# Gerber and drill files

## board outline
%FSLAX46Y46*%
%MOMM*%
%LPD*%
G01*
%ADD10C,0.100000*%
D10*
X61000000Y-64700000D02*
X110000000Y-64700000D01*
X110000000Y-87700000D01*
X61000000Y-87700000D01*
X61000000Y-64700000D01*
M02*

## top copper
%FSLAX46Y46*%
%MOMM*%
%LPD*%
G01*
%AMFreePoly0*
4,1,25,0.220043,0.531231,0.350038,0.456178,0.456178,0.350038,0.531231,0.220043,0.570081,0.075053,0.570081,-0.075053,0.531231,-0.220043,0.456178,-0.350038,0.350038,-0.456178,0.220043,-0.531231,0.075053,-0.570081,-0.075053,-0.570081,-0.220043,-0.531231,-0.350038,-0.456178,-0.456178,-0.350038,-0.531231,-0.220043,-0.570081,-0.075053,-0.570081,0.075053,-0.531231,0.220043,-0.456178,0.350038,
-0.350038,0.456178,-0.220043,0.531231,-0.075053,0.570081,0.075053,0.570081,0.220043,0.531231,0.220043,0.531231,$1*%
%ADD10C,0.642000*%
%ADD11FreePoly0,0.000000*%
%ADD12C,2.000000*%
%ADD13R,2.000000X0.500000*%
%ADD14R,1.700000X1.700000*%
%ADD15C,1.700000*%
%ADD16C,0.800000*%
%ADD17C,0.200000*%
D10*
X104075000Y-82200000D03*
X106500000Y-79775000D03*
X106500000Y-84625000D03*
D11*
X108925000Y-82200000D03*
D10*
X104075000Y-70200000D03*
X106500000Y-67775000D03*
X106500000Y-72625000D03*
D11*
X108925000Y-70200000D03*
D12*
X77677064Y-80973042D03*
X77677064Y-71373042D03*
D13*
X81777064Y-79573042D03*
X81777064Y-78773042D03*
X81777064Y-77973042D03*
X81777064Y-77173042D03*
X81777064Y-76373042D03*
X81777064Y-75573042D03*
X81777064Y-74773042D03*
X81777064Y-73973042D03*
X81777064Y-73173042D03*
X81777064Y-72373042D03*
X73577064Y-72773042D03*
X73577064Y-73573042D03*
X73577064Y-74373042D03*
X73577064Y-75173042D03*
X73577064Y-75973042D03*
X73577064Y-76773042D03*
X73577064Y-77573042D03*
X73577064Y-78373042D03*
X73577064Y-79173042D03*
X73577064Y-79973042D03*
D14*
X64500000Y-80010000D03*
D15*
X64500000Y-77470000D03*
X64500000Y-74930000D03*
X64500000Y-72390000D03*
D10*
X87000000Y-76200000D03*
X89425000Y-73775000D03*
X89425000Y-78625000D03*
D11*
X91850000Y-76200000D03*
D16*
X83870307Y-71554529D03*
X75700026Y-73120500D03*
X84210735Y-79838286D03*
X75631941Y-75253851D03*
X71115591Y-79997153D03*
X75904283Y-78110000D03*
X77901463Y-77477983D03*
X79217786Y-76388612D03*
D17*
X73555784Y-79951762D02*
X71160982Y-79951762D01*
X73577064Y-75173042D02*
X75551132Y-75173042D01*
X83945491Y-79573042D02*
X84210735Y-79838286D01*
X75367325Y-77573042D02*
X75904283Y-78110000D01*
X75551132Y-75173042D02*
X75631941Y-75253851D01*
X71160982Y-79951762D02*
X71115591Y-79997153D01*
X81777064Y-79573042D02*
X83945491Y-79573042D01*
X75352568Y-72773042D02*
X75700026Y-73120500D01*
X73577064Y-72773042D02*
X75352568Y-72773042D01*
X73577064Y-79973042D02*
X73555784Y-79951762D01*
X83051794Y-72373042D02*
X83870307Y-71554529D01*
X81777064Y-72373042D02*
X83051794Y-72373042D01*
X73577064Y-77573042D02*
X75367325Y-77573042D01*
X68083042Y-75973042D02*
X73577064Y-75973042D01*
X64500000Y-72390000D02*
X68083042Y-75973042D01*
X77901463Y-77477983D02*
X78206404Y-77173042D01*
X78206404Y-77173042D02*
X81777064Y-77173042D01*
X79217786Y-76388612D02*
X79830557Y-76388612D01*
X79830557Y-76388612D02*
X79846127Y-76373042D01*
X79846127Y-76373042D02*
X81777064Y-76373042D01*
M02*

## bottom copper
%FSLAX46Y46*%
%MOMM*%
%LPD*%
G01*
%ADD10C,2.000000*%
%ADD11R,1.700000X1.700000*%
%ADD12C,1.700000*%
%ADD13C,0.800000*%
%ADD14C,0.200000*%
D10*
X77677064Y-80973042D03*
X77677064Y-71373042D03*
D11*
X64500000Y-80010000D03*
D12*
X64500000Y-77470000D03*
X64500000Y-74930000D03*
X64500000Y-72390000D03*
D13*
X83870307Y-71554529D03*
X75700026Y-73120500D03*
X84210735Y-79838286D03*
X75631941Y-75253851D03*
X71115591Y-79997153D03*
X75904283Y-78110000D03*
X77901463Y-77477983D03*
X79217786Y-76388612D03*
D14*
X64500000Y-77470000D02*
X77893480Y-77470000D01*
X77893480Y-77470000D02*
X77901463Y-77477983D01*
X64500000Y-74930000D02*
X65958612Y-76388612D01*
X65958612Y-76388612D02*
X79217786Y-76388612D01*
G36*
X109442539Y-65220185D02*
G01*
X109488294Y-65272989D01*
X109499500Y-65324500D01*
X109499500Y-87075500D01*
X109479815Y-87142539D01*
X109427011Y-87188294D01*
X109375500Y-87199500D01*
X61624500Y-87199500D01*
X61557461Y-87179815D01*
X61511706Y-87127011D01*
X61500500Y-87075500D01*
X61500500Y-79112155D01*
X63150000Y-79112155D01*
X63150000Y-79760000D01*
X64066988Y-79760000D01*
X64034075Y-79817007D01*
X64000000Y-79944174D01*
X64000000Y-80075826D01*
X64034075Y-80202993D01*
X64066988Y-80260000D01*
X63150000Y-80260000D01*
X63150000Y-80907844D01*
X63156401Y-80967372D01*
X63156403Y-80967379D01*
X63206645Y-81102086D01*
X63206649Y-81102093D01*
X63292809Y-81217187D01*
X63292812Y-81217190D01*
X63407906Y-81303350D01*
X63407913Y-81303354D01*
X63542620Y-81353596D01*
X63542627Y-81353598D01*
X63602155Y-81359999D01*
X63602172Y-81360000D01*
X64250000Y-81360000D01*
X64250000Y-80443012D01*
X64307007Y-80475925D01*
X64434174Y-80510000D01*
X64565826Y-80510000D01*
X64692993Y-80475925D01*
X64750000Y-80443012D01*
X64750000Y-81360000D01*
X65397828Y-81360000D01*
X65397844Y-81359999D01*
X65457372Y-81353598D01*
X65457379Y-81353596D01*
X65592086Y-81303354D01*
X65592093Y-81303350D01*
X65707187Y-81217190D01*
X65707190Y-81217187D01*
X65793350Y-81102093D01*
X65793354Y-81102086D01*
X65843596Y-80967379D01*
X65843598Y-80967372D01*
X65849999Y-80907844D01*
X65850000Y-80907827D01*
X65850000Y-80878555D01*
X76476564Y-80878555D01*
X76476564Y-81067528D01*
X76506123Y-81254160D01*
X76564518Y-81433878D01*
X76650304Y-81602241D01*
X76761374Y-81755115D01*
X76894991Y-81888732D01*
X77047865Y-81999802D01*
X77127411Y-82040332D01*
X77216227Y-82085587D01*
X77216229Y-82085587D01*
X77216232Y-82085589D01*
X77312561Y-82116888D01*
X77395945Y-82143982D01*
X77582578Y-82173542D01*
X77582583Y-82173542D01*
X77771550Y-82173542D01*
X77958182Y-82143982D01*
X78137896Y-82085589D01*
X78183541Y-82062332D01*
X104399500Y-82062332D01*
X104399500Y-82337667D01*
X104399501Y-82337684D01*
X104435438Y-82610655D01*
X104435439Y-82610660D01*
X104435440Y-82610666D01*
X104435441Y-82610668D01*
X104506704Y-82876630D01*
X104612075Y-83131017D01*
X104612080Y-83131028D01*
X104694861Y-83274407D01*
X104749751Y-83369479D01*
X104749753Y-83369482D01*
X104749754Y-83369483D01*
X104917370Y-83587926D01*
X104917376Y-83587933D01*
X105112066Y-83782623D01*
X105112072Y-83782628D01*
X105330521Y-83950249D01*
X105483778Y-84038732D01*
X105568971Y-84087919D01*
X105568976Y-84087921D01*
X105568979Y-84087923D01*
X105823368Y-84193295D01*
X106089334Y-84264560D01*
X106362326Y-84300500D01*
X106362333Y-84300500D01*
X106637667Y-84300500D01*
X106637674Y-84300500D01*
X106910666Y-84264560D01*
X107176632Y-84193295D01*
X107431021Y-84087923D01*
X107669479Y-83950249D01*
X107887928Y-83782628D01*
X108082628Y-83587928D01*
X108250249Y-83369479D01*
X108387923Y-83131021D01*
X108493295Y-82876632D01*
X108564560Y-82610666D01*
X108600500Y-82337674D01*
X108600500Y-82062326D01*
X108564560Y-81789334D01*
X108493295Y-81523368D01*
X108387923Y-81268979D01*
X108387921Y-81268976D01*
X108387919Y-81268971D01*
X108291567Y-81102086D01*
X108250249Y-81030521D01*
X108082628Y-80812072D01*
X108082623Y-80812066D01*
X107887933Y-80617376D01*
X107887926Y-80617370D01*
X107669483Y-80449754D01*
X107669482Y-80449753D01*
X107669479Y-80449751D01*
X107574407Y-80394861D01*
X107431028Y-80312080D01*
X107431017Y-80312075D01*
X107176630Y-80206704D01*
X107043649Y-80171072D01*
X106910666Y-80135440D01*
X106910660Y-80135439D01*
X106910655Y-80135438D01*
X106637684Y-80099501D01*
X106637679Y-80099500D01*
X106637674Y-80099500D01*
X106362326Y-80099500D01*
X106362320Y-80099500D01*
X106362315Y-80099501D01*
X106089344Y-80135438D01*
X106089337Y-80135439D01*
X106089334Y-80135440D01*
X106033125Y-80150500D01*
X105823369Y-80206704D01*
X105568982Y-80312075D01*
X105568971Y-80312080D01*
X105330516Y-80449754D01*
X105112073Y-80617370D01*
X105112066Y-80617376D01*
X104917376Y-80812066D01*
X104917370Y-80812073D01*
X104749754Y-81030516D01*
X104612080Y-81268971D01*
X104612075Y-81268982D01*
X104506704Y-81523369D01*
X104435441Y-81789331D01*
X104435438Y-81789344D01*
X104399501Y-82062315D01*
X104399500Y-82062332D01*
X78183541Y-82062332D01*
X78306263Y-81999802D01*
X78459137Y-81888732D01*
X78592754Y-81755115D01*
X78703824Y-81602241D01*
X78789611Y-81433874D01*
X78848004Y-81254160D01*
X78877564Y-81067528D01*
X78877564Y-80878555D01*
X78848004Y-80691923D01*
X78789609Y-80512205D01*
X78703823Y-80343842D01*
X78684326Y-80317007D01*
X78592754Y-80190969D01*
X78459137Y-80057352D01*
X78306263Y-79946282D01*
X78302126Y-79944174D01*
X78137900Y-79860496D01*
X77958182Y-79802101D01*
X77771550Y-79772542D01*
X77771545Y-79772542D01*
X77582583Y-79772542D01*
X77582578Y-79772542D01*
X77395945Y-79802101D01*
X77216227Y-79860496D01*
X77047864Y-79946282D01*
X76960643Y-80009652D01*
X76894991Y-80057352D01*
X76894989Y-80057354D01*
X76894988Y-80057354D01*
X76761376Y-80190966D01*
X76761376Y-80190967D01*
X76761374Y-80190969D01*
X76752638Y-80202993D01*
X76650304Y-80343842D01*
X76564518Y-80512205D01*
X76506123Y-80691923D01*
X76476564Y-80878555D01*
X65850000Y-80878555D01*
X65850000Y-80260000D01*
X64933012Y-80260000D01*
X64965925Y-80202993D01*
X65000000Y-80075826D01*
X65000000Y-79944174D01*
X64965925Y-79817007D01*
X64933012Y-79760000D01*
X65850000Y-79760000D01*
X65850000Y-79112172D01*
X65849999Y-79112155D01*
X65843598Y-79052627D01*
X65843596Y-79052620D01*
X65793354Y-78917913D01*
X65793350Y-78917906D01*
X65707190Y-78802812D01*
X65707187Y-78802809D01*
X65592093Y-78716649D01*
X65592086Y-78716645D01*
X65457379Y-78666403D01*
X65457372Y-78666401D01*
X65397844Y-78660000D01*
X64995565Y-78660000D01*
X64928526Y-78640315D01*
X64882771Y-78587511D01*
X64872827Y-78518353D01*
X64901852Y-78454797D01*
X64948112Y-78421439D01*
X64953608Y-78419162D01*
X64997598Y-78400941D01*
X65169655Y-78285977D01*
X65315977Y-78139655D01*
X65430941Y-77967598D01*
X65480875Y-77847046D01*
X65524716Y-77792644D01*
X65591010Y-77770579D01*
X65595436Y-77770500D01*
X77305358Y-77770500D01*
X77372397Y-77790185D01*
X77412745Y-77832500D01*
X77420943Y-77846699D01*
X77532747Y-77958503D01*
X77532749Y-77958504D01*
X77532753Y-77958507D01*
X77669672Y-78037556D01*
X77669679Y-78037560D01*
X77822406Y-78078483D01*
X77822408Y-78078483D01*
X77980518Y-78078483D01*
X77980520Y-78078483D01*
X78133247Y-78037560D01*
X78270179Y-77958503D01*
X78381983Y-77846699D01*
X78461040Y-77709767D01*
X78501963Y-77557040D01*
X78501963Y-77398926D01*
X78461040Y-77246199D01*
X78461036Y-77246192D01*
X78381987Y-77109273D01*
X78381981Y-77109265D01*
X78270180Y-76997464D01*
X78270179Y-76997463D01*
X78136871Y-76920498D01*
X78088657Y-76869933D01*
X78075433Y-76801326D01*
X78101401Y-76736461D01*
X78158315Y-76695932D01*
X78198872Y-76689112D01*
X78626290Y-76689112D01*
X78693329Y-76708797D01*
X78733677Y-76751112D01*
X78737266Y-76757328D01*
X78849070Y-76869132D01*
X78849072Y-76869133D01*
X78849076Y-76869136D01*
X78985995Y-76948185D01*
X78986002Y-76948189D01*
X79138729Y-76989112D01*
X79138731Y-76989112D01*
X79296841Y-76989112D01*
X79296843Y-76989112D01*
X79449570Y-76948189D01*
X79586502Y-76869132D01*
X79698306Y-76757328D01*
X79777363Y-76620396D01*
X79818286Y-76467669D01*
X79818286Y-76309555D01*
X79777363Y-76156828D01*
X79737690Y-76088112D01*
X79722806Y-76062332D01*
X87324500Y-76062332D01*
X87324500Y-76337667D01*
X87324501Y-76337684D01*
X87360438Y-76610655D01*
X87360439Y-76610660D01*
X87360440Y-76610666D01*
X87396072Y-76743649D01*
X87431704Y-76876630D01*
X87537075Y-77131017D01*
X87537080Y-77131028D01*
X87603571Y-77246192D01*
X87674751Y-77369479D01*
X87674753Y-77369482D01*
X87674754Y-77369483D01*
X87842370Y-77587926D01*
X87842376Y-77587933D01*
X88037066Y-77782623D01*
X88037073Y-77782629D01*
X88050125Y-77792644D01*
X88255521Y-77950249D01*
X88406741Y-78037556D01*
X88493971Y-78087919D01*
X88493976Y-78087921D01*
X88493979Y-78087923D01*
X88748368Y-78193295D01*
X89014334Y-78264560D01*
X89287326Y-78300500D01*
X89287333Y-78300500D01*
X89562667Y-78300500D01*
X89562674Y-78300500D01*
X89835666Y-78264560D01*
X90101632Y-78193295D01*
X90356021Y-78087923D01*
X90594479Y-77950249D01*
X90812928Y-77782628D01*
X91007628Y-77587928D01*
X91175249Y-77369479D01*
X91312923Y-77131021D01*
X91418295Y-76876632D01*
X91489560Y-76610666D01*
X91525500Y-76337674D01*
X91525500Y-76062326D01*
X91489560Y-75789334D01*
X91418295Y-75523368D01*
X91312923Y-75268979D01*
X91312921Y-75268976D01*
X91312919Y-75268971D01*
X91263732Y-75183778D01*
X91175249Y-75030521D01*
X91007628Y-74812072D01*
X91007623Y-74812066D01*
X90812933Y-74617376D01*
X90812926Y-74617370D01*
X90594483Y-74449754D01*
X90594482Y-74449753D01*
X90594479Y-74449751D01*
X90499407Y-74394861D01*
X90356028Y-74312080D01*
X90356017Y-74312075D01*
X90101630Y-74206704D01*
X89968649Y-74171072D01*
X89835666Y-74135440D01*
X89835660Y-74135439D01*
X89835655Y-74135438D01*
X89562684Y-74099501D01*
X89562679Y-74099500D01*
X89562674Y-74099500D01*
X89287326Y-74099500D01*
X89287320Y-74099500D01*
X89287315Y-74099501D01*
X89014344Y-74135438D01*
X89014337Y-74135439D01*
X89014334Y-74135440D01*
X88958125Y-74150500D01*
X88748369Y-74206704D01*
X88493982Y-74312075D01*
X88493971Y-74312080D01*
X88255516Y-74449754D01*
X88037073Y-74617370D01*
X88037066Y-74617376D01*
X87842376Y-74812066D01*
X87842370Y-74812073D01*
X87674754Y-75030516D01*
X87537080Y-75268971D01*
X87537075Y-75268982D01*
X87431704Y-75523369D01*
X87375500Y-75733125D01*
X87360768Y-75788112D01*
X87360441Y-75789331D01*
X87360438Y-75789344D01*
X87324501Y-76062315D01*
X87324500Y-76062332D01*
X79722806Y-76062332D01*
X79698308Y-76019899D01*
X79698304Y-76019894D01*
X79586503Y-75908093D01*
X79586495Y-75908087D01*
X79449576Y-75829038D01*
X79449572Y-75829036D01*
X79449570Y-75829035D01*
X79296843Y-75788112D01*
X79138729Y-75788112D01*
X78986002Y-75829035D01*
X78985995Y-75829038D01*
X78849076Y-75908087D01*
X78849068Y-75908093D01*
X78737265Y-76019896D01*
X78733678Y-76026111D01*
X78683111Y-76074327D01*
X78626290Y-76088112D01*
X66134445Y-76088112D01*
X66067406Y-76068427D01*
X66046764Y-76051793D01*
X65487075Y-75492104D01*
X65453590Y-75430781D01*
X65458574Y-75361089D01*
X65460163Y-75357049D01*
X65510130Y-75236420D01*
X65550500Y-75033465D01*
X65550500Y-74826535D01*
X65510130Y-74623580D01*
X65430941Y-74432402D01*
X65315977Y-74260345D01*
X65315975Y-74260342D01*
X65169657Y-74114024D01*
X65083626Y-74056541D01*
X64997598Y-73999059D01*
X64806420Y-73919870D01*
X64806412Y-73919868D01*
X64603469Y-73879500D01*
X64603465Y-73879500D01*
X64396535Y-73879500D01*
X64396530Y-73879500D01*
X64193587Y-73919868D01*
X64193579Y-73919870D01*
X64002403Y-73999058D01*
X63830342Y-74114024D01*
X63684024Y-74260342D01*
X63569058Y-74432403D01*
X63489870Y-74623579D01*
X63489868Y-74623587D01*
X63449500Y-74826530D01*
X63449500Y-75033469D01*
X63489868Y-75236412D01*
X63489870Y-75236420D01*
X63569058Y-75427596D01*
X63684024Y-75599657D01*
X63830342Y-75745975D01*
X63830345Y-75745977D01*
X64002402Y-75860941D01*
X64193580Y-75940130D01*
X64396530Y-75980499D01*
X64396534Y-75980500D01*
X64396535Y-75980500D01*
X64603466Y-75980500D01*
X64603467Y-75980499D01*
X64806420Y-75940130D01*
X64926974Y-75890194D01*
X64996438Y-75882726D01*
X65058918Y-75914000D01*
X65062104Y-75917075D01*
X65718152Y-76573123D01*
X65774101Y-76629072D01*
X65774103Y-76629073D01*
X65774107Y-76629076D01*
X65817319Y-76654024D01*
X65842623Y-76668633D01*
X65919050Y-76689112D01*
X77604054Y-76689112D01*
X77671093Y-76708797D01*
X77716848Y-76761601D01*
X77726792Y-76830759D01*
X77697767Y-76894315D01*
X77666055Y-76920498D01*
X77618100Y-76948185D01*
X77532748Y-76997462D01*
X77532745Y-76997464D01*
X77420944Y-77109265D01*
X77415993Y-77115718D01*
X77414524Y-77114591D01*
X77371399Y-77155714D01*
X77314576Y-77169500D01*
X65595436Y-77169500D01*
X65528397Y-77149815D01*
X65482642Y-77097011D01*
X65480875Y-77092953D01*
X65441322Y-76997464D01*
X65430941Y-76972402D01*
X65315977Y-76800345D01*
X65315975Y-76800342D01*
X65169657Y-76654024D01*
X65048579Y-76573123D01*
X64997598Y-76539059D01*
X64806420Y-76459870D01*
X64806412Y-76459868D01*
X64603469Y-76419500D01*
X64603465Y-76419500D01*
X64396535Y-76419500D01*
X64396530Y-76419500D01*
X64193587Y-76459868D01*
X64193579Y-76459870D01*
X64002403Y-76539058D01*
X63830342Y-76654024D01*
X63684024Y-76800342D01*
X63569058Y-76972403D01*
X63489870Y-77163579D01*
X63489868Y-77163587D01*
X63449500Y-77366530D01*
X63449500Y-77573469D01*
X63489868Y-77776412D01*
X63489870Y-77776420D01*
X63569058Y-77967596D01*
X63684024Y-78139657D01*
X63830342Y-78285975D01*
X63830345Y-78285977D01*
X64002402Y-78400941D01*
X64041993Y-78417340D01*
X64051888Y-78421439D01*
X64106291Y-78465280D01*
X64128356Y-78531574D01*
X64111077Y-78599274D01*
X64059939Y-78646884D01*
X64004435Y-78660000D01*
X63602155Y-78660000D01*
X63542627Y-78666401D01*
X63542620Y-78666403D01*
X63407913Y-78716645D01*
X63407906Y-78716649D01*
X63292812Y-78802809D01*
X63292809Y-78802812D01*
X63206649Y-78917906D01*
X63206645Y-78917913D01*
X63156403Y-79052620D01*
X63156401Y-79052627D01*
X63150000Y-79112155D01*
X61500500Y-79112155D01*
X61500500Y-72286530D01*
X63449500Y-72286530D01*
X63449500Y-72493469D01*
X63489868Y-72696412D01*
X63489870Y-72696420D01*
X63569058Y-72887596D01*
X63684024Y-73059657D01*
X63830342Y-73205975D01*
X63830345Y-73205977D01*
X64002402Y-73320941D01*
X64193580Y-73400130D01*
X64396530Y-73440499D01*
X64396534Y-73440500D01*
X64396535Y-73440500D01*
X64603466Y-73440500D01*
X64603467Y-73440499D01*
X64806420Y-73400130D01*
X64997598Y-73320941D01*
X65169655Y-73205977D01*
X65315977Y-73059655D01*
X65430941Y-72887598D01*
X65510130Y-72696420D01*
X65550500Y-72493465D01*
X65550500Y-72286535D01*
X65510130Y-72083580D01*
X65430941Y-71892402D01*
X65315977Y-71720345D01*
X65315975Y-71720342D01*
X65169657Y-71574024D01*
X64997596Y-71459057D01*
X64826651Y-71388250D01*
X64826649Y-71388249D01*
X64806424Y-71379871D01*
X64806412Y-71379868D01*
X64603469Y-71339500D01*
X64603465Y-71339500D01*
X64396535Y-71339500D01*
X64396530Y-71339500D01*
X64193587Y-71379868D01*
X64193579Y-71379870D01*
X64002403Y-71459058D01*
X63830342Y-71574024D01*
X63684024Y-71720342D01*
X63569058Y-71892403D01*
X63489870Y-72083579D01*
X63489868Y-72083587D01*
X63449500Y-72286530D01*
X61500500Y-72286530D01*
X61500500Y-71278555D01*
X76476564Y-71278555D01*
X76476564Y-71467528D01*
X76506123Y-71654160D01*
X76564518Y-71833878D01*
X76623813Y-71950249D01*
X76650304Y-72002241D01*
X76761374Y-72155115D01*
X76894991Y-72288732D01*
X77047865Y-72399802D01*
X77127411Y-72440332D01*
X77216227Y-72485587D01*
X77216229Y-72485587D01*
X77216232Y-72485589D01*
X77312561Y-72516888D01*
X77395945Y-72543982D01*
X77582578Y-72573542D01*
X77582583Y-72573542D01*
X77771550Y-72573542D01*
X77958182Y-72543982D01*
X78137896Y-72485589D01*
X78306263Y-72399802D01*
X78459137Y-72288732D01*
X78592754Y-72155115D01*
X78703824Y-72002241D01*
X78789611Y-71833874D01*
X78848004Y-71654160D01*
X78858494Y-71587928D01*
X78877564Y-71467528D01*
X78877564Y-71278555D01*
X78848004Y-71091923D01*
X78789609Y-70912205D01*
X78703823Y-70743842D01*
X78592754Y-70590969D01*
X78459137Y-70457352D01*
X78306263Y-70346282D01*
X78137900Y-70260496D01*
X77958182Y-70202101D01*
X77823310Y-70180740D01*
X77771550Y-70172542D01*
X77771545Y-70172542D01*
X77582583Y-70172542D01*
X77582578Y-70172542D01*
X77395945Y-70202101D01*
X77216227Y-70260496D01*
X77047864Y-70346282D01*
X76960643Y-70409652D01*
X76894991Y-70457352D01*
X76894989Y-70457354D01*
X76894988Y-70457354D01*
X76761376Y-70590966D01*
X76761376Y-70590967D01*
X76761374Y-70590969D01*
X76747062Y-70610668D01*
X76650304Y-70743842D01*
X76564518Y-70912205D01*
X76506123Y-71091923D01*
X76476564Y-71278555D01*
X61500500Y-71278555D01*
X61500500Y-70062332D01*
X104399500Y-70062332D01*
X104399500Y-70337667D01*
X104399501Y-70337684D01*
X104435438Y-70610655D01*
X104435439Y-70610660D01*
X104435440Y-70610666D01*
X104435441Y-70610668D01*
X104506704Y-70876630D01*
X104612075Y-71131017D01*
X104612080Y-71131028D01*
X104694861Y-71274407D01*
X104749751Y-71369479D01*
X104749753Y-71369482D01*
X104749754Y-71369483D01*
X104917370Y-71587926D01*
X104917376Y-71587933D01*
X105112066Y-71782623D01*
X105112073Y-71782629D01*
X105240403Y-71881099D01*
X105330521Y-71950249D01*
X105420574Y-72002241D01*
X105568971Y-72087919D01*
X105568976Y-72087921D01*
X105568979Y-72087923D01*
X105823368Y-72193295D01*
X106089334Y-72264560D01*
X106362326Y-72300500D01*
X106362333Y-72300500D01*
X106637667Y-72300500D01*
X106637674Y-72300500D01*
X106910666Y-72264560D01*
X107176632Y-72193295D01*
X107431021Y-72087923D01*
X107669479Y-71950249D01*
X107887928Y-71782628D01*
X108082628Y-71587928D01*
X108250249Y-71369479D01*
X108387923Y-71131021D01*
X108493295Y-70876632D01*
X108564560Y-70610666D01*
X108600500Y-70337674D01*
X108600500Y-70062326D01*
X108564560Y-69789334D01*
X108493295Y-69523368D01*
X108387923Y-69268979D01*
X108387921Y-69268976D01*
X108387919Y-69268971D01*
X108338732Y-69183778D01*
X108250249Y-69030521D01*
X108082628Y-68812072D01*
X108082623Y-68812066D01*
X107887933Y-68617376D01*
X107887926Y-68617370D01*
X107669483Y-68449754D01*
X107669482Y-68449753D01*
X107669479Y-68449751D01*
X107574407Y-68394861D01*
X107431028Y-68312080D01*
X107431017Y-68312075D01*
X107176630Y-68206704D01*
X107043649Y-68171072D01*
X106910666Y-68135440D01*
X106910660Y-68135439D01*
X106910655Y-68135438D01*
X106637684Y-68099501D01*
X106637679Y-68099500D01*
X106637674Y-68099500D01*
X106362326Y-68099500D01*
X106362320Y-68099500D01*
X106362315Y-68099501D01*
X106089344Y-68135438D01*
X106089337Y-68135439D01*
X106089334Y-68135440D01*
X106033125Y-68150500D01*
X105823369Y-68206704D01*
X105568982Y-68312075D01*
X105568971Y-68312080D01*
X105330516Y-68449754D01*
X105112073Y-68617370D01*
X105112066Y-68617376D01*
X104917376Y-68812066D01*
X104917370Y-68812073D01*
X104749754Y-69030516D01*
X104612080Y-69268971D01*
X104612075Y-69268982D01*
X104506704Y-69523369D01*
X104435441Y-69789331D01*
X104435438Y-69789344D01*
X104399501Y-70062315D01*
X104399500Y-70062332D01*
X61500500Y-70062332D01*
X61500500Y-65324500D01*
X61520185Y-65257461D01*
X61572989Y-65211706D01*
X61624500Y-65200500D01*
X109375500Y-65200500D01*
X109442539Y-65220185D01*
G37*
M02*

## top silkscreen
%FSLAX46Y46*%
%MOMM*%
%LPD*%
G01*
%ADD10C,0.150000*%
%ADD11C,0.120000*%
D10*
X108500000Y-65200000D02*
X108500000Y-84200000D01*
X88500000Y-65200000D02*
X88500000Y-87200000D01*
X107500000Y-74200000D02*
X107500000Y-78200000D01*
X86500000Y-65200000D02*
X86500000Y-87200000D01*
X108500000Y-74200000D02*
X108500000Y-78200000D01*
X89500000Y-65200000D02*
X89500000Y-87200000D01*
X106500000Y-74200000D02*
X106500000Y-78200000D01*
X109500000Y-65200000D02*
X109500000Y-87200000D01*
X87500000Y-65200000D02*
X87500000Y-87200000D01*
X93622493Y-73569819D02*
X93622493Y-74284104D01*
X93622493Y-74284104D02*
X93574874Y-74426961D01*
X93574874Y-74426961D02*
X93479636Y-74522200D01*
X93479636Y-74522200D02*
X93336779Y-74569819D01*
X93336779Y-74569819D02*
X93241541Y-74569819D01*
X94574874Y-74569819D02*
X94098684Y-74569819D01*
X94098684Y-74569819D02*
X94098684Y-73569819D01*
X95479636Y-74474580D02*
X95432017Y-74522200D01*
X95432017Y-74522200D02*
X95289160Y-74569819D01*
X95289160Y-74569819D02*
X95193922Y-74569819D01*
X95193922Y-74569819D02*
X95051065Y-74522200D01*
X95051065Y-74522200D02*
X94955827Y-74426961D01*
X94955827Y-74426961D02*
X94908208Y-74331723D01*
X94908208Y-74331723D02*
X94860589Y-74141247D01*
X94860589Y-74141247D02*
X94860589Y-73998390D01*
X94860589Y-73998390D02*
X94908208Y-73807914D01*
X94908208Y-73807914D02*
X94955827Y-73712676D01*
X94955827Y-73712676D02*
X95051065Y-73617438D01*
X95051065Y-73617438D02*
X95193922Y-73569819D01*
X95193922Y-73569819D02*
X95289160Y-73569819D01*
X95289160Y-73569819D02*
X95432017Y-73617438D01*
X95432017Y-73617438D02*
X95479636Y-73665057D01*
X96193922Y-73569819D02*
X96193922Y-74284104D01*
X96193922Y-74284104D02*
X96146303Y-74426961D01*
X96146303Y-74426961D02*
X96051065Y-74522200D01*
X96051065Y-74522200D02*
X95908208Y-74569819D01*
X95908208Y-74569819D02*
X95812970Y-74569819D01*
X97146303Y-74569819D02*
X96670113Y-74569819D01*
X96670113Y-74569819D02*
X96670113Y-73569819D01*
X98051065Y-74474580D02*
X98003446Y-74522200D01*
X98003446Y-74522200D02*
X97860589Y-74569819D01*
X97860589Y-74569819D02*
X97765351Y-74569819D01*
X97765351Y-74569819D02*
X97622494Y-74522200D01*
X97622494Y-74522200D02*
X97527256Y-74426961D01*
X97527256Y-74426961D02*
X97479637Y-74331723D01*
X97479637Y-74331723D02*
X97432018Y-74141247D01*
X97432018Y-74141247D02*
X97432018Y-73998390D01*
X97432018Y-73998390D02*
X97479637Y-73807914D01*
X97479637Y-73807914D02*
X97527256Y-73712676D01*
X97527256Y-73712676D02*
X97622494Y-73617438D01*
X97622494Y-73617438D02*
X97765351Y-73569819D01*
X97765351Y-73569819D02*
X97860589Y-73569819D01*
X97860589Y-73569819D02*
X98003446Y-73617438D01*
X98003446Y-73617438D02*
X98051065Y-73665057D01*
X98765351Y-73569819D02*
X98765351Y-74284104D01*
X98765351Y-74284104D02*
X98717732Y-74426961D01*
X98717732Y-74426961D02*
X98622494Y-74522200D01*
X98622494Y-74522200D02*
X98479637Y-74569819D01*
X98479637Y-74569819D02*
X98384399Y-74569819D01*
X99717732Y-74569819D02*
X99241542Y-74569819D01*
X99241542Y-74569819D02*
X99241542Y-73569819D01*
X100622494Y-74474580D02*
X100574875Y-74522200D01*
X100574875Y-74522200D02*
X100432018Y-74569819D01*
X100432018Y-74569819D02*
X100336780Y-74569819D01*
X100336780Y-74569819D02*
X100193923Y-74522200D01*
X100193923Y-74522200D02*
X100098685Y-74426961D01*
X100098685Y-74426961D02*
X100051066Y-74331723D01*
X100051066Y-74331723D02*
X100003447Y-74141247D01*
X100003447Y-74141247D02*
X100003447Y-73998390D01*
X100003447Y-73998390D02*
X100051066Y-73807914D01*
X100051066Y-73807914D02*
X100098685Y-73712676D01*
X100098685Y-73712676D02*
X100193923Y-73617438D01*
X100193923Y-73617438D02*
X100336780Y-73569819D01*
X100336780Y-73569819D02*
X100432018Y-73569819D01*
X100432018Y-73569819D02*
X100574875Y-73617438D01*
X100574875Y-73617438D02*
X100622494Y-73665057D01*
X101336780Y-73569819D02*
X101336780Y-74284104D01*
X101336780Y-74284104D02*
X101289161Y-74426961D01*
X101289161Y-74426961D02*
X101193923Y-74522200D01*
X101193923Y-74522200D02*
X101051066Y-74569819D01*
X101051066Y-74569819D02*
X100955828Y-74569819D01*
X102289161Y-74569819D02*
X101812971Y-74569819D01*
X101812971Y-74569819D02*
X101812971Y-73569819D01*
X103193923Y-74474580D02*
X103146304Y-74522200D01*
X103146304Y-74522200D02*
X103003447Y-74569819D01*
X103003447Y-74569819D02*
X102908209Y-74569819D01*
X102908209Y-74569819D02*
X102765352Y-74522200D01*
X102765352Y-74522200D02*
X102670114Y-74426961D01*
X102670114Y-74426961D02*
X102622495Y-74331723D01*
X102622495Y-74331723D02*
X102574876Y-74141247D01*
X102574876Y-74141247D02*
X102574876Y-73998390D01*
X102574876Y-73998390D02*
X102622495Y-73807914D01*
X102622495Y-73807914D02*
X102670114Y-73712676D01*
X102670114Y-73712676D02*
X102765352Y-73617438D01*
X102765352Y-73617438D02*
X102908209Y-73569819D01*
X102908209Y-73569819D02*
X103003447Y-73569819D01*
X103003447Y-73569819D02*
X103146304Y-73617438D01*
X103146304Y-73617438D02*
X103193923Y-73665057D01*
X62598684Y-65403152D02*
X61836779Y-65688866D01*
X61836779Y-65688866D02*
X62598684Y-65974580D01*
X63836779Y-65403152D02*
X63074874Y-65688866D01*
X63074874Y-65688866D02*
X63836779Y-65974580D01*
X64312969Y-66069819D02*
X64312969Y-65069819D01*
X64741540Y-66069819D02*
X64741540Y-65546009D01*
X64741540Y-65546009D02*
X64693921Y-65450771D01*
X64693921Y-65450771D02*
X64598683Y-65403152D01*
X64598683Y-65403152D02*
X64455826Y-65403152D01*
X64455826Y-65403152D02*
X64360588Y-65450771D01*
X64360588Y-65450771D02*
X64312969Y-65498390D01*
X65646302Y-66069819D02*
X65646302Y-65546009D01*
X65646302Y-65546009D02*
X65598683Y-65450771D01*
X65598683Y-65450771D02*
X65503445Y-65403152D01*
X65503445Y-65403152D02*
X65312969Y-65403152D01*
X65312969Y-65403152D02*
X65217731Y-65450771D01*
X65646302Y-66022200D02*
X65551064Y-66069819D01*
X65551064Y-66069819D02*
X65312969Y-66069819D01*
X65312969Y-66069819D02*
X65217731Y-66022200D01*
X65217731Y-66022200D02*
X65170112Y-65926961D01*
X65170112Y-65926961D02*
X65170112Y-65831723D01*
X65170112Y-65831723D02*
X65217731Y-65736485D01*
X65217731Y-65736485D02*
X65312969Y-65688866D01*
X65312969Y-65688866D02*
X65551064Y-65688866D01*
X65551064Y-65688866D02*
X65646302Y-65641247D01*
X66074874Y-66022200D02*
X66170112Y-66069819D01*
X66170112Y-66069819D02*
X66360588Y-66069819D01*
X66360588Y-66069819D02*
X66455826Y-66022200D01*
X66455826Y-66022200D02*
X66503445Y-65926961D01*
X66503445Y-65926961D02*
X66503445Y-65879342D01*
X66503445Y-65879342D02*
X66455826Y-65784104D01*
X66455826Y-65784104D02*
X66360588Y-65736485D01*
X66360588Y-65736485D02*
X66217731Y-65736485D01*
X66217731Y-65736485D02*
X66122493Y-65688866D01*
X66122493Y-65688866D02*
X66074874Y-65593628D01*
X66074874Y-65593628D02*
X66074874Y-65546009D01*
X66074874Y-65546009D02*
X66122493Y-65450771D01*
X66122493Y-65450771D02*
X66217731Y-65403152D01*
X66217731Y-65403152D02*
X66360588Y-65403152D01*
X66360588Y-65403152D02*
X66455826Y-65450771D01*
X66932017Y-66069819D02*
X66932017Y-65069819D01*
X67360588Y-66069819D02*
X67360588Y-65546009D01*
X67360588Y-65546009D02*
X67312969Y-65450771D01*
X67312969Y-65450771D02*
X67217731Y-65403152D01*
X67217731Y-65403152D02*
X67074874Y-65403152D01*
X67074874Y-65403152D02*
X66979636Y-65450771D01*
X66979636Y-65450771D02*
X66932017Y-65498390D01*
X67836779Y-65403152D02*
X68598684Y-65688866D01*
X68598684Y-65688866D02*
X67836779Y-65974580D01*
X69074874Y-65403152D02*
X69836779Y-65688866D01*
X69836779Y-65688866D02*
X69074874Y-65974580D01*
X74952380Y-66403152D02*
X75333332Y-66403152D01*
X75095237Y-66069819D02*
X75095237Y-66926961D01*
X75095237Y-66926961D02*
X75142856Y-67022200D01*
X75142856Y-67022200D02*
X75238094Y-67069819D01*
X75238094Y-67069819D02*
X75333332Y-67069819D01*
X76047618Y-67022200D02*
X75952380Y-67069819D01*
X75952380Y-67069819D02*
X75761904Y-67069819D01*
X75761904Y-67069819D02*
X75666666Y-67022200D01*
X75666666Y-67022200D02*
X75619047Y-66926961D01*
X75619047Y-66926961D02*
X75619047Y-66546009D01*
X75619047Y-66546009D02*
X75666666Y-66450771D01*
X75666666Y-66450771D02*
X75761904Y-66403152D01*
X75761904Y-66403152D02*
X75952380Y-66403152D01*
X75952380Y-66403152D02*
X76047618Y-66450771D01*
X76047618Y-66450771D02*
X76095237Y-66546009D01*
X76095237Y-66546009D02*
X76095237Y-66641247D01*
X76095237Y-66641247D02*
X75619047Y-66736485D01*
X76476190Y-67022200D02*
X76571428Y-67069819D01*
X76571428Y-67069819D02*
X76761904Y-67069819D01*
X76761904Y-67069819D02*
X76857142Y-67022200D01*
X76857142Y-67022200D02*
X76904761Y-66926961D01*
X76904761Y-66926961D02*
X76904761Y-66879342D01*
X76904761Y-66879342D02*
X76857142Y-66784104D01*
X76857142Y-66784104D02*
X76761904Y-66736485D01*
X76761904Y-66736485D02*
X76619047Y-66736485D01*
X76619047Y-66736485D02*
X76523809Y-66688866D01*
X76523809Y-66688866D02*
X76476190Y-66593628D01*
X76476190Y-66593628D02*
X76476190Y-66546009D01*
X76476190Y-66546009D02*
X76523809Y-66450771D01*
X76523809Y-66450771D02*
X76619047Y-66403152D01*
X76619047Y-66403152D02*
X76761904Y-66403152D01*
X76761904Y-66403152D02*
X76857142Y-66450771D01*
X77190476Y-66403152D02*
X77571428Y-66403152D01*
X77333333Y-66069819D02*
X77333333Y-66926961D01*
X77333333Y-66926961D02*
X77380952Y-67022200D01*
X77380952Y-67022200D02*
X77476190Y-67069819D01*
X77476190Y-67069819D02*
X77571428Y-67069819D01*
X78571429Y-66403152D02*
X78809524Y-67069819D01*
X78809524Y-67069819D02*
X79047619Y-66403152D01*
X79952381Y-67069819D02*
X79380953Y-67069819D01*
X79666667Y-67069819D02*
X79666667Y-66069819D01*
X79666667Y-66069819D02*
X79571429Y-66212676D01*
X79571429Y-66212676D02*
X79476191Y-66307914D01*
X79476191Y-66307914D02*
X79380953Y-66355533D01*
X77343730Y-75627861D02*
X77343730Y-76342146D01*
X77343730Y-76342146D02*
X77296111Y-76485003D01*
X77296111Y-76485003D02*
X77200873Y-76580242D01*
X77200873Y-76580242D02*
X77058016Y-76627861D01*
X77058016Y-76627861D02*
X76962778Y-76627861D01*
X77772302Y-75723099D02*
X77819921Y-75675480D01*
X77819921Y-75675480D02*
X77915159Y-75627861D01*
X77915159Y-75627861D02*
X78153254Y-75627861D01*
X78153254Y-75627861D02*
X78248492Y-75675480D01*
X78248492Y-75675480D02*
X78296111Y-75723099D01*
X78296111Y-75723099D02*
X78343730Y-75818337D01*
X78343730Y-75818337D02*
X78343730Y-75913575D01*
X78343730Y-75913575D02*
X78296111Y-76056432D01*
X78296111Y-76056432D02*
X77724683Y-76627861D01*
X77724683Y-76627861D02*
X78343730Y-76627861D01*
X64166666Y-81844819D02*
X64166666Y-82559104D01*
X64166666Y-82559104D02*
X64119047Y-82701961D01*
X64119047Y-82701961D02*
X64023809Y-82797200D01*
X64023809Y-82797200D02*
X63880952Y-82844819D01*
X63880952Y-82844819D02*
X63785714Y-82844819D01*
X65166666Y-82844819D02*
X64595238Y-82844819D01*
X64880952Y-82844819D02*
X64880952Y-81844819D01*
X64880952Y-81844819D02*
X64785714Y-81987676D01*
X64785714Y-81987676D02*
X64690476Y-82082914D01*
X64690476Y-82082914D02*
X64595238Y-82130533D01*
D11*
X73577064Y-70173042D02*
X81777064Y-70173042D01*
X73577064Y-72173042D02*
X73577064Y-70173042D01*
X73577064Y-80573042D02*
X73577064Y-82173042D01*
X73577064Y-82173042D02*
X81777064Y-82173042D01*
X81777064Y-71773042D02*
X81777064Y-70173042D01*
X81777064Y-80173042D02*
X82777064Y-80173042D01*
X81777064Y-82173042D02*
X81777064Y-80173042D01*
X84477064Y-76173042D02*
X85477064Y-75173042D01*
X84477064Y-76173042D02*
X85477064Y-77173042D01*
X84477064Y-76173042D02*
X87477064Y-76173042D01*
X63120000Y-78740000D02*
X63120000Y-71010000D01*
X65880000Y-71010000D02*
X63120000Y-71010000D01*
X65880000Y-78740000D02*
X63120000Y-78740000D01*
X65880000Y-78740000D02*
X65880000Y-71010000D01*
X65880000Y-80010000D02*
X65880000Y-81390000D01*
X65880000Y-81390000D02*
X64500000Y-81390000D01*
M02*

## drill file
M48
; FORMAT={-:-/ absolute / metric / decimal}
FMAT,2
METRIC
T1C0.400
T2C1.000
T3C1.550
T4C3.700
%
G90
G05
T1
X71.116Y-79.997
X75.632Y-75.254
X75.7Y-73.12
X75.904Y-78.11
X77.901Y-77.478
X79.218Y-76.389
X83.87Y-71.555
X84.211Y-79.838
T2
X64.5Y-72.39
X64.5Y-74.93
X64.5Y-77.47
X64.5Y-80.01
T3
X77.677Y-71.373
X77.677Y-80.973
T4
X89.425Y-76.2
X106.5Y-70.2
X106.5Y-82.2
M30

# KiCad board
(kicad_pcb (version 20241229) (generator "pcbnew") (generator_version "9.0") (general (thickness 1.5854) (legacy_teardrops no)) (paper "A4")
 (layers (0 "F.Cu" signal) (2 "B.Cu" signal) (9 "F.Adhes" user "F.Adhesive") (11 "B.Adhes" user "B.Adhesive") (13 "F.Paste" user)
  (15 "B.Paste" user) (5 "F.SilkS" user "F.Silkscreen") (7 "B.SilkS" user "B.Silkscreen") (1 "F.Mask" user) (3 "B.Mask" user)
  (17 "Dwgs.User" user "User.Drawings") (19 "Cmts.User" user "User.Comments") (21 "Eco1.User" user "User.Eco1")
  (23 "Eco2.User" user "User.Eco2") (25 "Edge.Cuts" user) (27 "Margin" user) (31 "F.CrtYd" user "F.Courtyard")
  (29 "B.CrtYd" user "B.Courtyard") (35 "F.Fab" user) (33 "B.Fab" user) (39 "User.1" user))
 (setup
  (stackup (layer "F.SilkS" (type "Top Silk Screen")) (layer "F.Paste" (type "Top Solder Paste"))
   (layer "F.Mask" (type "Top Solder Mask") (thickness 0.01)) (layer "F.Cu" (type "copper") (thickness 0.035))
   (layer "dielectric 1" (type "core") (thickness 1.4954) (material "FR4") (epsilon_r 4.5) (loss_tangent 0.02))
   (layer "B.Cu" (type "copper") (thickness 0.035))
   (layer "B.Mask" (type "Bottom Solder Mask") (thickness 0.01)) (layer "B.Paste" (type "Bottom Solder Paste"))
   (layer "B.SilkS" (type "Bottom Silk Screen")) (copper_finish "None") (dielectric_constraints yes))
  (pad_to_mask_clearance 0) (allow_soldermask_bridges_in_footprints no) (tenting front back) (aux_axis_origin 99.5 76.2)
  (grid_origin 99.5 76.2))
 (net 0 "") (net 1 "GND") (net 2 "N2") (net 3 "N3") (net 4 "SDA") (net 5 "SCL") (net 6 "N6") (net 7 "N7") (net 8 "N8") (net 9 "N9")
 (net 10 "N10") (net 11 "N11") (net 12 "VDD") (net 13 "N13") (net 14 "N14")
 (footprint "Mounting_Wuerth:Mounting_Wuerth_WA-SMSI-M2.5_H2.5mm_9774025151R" (layer "F.Cu") (at 106.5 82.2)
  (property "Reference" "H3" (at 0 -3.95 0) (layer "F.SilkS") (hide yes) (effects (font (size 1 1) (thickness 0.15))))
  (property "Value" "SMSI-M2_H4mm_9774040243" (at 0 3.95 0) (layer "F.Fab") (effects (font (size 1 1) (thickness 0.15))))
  (pad "" smd custom (at -1.704127 -1.704127) (size 0.51 0.51) (layers "F.Paste") (options (clearance outline) (anchor circle)) (primitives))
  (pad "" smd custom (at -1.704127 1.704127) (size 0.51 0.51) (layers "F.Paste") (options (clearance outline) (anchor circle)) (primitives))
  (pad "" np_thru_hole circle (at 0 0) (size 3.7 3.7) (drill 3.7) (layers "*.Cu" "*.Mask"))
  (pad "" smd custom (at 1.704127 -1.704127) (size 0.51 0.51) (layers "F.Paste") (options (clearance outline) (anchor circle)) (primitives))
  (pad "" smd custom (at 1.704127 1.704127) (size 0.51 0.51) (layers "F.Paste") (options (clearance outline) (anchor circle)) (primitives))
  (pad "1" smd circle (at -2.425 0) (size 0.642 0.642) (layers "F.Cu"))
  (pad "1" smd circle (at 0 -2.425) (size 0.642 0.642) (layers "F.Cu"))
  (pad "1" smd circle (at 0 2.425) (size 0.642 0.642) (layers "F.Cu"))
  (pad "1" smd custom (at 2.425 0) (size 1.15 1.15) (layers "F.Cu" "F.Mask") (options (clearance outline) (anchor circle)) (primitives)))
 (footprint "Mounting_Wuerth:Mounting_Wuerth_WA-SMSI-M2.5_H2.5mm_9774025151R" (layer "F.Cu") (at 106.5 70.2)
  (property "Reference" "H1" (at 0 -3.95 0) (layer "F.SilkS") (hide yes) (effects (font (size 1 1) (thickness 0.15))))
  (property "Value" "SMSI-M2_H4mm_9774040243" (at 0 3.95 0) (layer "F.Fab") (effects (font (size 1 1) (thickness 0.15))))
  (pad "" smd custom (at -1.704127 -1.704127) (size 0.51 0.51) (layers "F.Paste") (options (clearance outline) (anchor circle)) (primitives))
  (pad "" smd custom (at -1.704127 1.704127) (size 0.51 0.51) (layers "F.Paste") (options (clearance outline) (anchor circle)) (primitives))
  (pad "" np_thru_hole circle (at 0 0) (size 3.7 3.7) (drill 3.7) (layers "*.Cu" "*.Mask"))
  (pad "" smd custom (at 1.704127 -1.704127) (size 0.51 0.51) (layers "F.Paste") (options (clearance outline) (anchor circle)) (primitives))
  (pad "" smd custom (at 1.704127 1.704127) (size 0.51 0.51) (layers "F.Paste") (options (clearance outline) (anchor circle)) (primitives))
  (pad "1" smd circle (at -2.425 0) (size 0.642 0.642) (layers "F.Cu"))
  (pad "1" smd circle (at 0 -2.425) (size 0.642 0.642) (layers "F.Cu"))
  (pad "1" smd circle (at 0 2.425) (size 0.642 0.642) (layers "F.Cu"))
  (pad "1" smd custom (at 2.425 0) (size 1.15 1.15) (layers "F.Cu" "F.Mask") (options (clearance outline) (anchor circle)) (primitives)))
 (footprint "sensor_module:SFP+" (layer "F.Cu") (at 71.477064 76.173042 180)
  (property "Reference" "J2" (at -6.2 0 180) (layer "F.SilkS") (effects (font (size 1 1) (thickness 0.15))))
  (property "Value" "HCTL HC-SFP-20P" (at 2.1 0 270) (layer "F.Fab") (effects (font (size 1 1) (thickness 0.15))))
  (fp_line (start -2.1 6) (end -10.3 6) (stroke (width 0.12) (type solid)) (layer "F.SilkS"))
  (fp_line (start -2.1 4) (end -2.1 6) (stroke (width 0.12) (type solid)) (layer "F.SilkS"))
  (fp_line (start -2.1 -4.4) (end -2.1 -6) (stroke (width 0.12) (type solid)) (layer "F.SilkS"))
  (fp_line (start -2.1 -6) (end -10.3 -6) (stroke (width 0.12) (type solid)) (layer "F.SilkS"))
  (fp_line (start -10.3 4.4) (end -10.3 6) (stroke (width 0.12) (type solid)) (layer "F.SilkS"))
  (fp_line (start -10.3 -4) (end -11.3 -4) (stroke (width 0.12) (type solid)) (layer "F.SilkS"))
  (fp_line (start -10.3 -6) (end -10.3 -4) (stroke (width 0.12) (type solid)) (layer "F.SilkS"))
  (fp_line (start -13 0) (end -14 1) (stroke (width 0.12) (type solid)) (layer "F.SilkS"))
  (fp_line (start -13 0) (end -14 -1) (stroke (width 0.12) (type solid)) (layer "F.SilkS"))
  (fp_line (start -13 0) (end -16 0) (stroke (width 0.12) (type solid)) (layer "F.SilkS"))
  (pad "" np_thru_hole circle (at -6.2 -4.8 180) (size 2 2) (drill 1.55) (layers "*.Cu" "*.Mask"))
  (pad "" np_thru_hole circle (at -6.2 4.8 180) (size 2 2) (drill 1.55) (layers "*.Cu" "*.Mask"))
  (pad "1" smd rect (at -10.3 -3.4 180) (size 2 0.5) (layers "F.Cu" "F.Mask" "F.Paste") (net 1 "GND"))
  (pad "2" smd rect (at -10.3 -2.6 180) (size 2 0.5) (layers "F.Cu" "F.Mask" "F.Paste") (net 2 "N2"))
  (pad "3" smd rect (at -10.3 -1.8 180) (size 2 0.5) (layers "F.Cu" "F.Mask" "F.Paste") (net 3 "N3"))
  (pad "4" smd rect (at -10.3 -1 180) (size 2 0.5) (layers "F.Cu" "F.Mask" "F.Paste") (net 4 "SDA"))
  (pad "5" smd rect (at -10.3 -0.2 180) (size 2 0.5) (layers "F.Cu" "F.Mask" "F.Paste") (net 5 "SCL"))
  (pad "6" smd rect (at -10.3 0.6 180) (size 2 0.5) (layers "F.Cu" "F.Mask" "F.Paste") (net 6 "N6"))
  (pad "7" smd rect (at -10.3 1.4 180) (size 2 0.5) (layers "F.Cu" "F.Mask" "F.Paste") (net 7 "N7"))
  (pad "8" smd rect (at -10.3 2.2 180) (size 2 0.5) (layers "F.Cu" "F.Mask" "F.Paste") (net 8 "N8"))
  (pad "9" smd rect (at -10.3 3 180) (size 2 0.5) (layers "F.Cu" "F.Mask" "F.Paste") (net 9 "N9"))
  (pad "10" smd rect (at -10.3 3.8 180) (size 2 0.5) (layers "F.Cu" "F.Mask" "F.Paste") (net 1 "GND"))
  (pad "11" smd rect (at -2.1 3.4 180) (size 2 0.5) (layers "F.Cu" "F.Mask" "F.Paste") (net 1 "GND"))
  (pad "12" smd rect (at -2.1 2.6 180) (size 2 0.5) (layers "F.Cu" "F.Mask" "F.Paste") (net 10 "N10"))
  (pad "13" smd rect (at -2.1 1.8 180) (size 2 0.5) (layers "F.Cu" "F.Mask" "F.Paste") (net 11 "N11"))
  (pad "14" smd rect (at -2.1 1 180) (size 2 0.5) (layers "F.Cu" "F.Mask" "F.Paste") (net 1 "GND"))
  (pad "15" smd rect (at -2.1 0.2 180) (size 2 0.5) (layers "F.Cu" "F.Mask" "F.Paste") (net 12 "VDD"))
  (pad "16" smd rect (at -2.1 -0.6 180) (size 2 0.5) (layers "F.Cu" "F.Mask" "F.Paste") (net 12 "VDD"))
  (pad "17" smd rect (at -2.1 -1.4 180) (size 2 0.5) (layers "F.Cu" "F.Mask" "F.Paste") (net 1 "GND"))
  (pad "18" smd rect (at -2.1 -2.2 180) (size 2 0.5) (layers "F.Cu" "F.Mask" "F.Paste") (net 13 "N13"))
  (pad "19" smd rect (at -2.1 -3 180) (size 2 0.5) (layers "F.Cu" "F.Mask" "F.Paste") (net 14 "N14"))
  (pad "20" smd rect (at -2.1 -3.8 180) (size 2 0.5) (layers "F.Cu" "F.Mask" "F.Paste") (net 1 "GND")))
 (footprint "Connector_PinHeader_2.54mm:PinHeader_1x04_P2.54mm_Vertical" (layer "F.Cu") (at 64.5 80.01 180)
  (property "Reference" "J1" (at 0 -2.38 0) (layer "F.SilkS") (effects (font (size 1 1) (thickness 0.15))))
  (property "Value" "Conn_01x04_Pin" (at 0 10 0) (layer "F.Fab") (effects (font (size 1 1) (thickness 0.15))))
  (fp_line (start 1.38 1.27) (end 1.38 9) (stroke (width 0.12) (type solid)) (layer "F.SilkS"))
  (fp_line (start -1.38 9) (end 1.38 9) (stroke (width 0.12) (type solid)) (layer "F.SilkS"))
  (fp_line (start -1.38 1.27) (end 1.38 1.27) (stroke (width 0.12) (type solid)) (layer "F.SilkS"))
  (fp_line (start -1.38 1.27) (end -1.38 9) (stroke (width 0.12) (type solid)) (layer "F.SilkS"))
  (fp_line (start -1.38 0) (end -1.38 -1.38) (stroke (width 0.12) (type solid)) (layer "F.SilkS"))
  (fp_line (start -1.38 -1.38) (end 0 -1.38) (stroke (width 0.12) (type solid)) (layer "F.SilkS"))
  (pad "1" thru_hole rect (at 0 0 180) (size 1.7 1.7) (drill 1) (layers "*.Cu" "*.Mask") (remove_unused_layers no) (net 1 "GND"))
  (pad "2" thru_hole circle (at 0 2.54 180) (size 1.7 1.7) (drill 1) (layers "*.Cu" "*.Mask") (remove_unused_layers no) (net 4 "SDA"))
  (pad "3" thru_hole circle (at 0 5.08 180) (size 1.7 1.7) (drill 1) (layers "*.Cu" "*.Mask") (remove_unused_layers no) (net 5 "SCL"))
  (pad "4" thru_hole circle (at 0 7.62 180) (size 1.7 1.7) (drill 1) (layers "*.Cu" "*.Mask") (remove_unused_layers no) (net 12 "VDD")))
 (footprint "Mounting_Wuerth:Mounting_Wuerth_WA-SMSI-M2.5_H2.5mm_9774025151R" (layer "F.Cu") (at 89.425 76.2)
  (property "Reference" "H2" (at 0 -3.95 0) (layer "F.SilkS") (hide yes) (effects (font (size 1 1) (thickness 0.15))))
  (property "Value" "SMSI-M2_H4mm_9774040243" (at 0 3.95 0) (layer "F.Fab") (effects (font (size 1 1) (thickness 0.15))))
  (pad "" smd custom (at -1.704127 -1.704127) (size 0.51 0.51) (layers "F.Paste") (options (clearance outline) (anchor circle)) (primitives))
  (pad "" smd custom (at -1.704127 1.704127) (size 0.51 0.51) (layers "F.Paste") (options (clearance outline) (anchor circle)) (primitives))
  (pad "" np_thru_hole circle (at 0 0) (size 3.7 3.7) (drill 3.7) (layers "*.Cu" "*.Mask"))
  (pad "" smd custom (at 1.704127 -1.704127) (size 0.51 0.51) (layers "F.Paste") (options (clearance outline) (anchor circle)) (primitives))
  (pad "" smd custom (at 1.704127 1.704127) (size 0.51 0.51) (layers "F.Paste") (options (clearance outline) (anchor circle)) (primitives))
  (pad "1" smd circle (at -2.425 0) (size 0.642 0.642) (layers "F.Cu"))
  (pad "1" smd circle (at 0 -2.425) (size 0.642 0.642) (layers "F.Cu"))
  (pad "1" smd circle (at 0 2.425) (size 0.642 0.642) (layers "F.Cu"))
  (pad "1" smd custom (at 2.425 0) (size 1.15 1.15) (layers "F.Cu" "F.Mask") (options (clearance outline) (anchor circle)) (primitives)))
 (gr_line (start 108.5 65.2) (end 108.5 84.2) (stroke (width 0.15) (type default)) (layer "F.SilkS"))
 (gr_line (start 88.5 65.2) (end 88.5 87.2) (stroke (width 0.15) (type default)) (layer "F.SilkS"))
 (gr_line (start 107.5 74.2) (end 107.5 78.2) (stroke (width 0.15) (type default)) (layer "F.SilkS"))
 (gr_line (start 86.5 65.2) (end 86.5 87.2) (stroke (width 0.15) (type default)) (layer "F.SilkS"))
 (gr_line (start 108.5 74.2) (end 108.5 78.2) (stroke (width 0.15) (type default)) (layer "F.SilkS"))
 (gr_line (start 89.5 65.2) (end 89.5 87.2) (stroke (width 0.15) (type default)) (layer "F.SilkS"))
 (gr_line (start 106.5 74.2) (end 106.5 78.2) (stroke (width 0.15) (type default)) (layer "F.SilkS"))
 (gr_line (start 109.5 65.2) (end 109.5 87.2) (stroke (width 0.15) (type default)) (layer "F.SilkS"))
 (gr_line (start 87.5 65.2) (end 87.5 87.2) (stroke (width 0.15) (type default)) (layer "F.SilkS"))
 (gr_rect (start 61 64.7) (end 110 87.7) (stroke (width 0.1) (type default)) (fill no) (layer "Edge.Cuts"))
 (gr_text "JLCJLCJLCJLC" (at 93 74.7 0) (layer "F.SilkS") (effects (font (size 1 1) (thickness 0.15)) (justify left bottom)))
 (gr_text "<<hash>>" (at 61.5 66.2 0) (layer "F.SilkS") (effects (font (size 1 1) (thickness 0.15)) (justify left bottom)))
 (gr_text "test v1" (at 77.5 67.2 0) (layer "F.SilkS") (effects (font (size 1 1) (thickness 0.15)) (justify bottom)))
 (segment (start 73.555784 79.951762) (end 71.160982 79.951762) (width 0.2) (layer "F.Cu") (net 1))
 (segment (start 73.577064 75.173042) (end 75.551132 75.173042) (width 0.2) (layer "F.Cu") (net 1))
 (segment (start 83.945491 79.573042) (end 84.210735 79.838286) (width 0.2) (layer "F.Cu") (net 1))
 (segment (start 75.367325 77.573042) (end 75.904283 78.11) (width 0.2) (layer "F.Cu") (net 1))
 (segment (start 75.551132 75.173042) (end 75.631941 75.253851) (width 0.2) (layer "F.Cu") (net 1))
 (segment (start 71.160982 79.951762) (end 71.115591 79.997153) (width 0.2) (layer "F.Cu") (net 1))
 (segment (start 81.777064 79.573042) (end 83.945491 79.573042) (width 0.2) (layer "F.Cu") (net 1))
 (segment (start 75.352568 72.773042) (end 75.700026 73.1205) (width 0.2) (layer "F.Cu") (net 1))
 (segment (start 73.577064 72.773042) (end 75.352568 72.773042) (width 0.2) (layer "F.Cu") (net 1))
 (segment (start 73.577064 79.973042) (end 73.555784 79.951762) (width 0.2) (layer "F.Cu") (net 1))
 (segment (start 83.051794 72.373042) (end 83.870307 71.554529) (width 0.2) (layer "F.Cu") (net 1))
 (segment (start 81.777064 72.373042) (end 83.051794 72.373042) (width 0.2) (layer "F.Cu") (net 1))
 (segment (start 73.577064 77.573042) (end 75.367325 77.573042) (width 0.2) (layer "F.Cu") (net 1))
 (via (at 83.870307 71.554529) (size 0.8) (drill 0.4) (layers "F.Cu" "B.Cu") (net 1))
 (via (at 75.700026 73.1205) (size 0.8) (drill 0.4) (layers "F.Cu" "B.Cu") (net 1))
 (via (at 84.210735 79.838286) (size 0.8) (drill 0.4) (layers "F.Cu" "B.Cu") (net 1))
 (via (at 75.631941 75.253851) (size 0.8) (drill 0.4) (layers "F.Cu" "B.Cu") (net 1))
 (via (at 71.115591 79.997153) (size 0.8) (drill 0.4) (layers "F.Cu" "B.Cu") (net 1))
 (via (at 75.904283 78.11) (size 0.8) (drill 0.4) (layers "F.Cu" "B.Cu") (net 1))
 (segment (start 68.083042 75.973042) (end 73.577064 75.973042) (width 0.2) (layer "F.Cu") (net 12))
 (segment (start 64.5 72.39) (end 68.083042 75.973042) (width 0.2) (layer "F.Cu") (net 12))
 (segment (start 77.901463 77.477983) (end 78.206404 77.173042) (width 0.2) (layer "F.Cu") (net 4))
 (segment (start 78.206404 77.173042) (end 81.777064 77.173042) (width 0.2) (layer "F.Cu") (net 4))
 (via (at 77.901463 77.477983) (size 0.8) (drill 0.4) (layers "F.Cu" "B.Cu") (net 4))
 (segment (start 64.5 77.47) (end 77.89348 77.47) (width 0.2) (layer "B.Cu") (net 4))
 (segment (start 77.89348 77.47) (end 77.901463 77.477983) (width 0.2) (layer "B.Cu") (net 4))
 (segment (start 79.217786 76.388612) (end 79.830557 76.388612) (width 0.2) (layer "F.Cu") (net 5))
 (segment (start 79.830557 76.388612) (end 79.846127 76.373042) (width 0.2) (layer "F.Cu") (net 5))
 (segment (start 79.846127 76.373042) (end 81.777064 76.373042) (width 0.2) (layer "F.Cu") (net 5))
 (via (at 79.217786 76.388612) (size 0.8) (drill 0.4) (layers "F.Cu" "B.Cu") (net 5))
 (segment (start 64.5 74.93) (end 65.958612 76.388612) (width 0.2) (layer "B.Cu") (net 5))
 (segment (start 65.958612 76.388612) (end 79.217786 76.388612) (width 0.2) (layer "B.Cu") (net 5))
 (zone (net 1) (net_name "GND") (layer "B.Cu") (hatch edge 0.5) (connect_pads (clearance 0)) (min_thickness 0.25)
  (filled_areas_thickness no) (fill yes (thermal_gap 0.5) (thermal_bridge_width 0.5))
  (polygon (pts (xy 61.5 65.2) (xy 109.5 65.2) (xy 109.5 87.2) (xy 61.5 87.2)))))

